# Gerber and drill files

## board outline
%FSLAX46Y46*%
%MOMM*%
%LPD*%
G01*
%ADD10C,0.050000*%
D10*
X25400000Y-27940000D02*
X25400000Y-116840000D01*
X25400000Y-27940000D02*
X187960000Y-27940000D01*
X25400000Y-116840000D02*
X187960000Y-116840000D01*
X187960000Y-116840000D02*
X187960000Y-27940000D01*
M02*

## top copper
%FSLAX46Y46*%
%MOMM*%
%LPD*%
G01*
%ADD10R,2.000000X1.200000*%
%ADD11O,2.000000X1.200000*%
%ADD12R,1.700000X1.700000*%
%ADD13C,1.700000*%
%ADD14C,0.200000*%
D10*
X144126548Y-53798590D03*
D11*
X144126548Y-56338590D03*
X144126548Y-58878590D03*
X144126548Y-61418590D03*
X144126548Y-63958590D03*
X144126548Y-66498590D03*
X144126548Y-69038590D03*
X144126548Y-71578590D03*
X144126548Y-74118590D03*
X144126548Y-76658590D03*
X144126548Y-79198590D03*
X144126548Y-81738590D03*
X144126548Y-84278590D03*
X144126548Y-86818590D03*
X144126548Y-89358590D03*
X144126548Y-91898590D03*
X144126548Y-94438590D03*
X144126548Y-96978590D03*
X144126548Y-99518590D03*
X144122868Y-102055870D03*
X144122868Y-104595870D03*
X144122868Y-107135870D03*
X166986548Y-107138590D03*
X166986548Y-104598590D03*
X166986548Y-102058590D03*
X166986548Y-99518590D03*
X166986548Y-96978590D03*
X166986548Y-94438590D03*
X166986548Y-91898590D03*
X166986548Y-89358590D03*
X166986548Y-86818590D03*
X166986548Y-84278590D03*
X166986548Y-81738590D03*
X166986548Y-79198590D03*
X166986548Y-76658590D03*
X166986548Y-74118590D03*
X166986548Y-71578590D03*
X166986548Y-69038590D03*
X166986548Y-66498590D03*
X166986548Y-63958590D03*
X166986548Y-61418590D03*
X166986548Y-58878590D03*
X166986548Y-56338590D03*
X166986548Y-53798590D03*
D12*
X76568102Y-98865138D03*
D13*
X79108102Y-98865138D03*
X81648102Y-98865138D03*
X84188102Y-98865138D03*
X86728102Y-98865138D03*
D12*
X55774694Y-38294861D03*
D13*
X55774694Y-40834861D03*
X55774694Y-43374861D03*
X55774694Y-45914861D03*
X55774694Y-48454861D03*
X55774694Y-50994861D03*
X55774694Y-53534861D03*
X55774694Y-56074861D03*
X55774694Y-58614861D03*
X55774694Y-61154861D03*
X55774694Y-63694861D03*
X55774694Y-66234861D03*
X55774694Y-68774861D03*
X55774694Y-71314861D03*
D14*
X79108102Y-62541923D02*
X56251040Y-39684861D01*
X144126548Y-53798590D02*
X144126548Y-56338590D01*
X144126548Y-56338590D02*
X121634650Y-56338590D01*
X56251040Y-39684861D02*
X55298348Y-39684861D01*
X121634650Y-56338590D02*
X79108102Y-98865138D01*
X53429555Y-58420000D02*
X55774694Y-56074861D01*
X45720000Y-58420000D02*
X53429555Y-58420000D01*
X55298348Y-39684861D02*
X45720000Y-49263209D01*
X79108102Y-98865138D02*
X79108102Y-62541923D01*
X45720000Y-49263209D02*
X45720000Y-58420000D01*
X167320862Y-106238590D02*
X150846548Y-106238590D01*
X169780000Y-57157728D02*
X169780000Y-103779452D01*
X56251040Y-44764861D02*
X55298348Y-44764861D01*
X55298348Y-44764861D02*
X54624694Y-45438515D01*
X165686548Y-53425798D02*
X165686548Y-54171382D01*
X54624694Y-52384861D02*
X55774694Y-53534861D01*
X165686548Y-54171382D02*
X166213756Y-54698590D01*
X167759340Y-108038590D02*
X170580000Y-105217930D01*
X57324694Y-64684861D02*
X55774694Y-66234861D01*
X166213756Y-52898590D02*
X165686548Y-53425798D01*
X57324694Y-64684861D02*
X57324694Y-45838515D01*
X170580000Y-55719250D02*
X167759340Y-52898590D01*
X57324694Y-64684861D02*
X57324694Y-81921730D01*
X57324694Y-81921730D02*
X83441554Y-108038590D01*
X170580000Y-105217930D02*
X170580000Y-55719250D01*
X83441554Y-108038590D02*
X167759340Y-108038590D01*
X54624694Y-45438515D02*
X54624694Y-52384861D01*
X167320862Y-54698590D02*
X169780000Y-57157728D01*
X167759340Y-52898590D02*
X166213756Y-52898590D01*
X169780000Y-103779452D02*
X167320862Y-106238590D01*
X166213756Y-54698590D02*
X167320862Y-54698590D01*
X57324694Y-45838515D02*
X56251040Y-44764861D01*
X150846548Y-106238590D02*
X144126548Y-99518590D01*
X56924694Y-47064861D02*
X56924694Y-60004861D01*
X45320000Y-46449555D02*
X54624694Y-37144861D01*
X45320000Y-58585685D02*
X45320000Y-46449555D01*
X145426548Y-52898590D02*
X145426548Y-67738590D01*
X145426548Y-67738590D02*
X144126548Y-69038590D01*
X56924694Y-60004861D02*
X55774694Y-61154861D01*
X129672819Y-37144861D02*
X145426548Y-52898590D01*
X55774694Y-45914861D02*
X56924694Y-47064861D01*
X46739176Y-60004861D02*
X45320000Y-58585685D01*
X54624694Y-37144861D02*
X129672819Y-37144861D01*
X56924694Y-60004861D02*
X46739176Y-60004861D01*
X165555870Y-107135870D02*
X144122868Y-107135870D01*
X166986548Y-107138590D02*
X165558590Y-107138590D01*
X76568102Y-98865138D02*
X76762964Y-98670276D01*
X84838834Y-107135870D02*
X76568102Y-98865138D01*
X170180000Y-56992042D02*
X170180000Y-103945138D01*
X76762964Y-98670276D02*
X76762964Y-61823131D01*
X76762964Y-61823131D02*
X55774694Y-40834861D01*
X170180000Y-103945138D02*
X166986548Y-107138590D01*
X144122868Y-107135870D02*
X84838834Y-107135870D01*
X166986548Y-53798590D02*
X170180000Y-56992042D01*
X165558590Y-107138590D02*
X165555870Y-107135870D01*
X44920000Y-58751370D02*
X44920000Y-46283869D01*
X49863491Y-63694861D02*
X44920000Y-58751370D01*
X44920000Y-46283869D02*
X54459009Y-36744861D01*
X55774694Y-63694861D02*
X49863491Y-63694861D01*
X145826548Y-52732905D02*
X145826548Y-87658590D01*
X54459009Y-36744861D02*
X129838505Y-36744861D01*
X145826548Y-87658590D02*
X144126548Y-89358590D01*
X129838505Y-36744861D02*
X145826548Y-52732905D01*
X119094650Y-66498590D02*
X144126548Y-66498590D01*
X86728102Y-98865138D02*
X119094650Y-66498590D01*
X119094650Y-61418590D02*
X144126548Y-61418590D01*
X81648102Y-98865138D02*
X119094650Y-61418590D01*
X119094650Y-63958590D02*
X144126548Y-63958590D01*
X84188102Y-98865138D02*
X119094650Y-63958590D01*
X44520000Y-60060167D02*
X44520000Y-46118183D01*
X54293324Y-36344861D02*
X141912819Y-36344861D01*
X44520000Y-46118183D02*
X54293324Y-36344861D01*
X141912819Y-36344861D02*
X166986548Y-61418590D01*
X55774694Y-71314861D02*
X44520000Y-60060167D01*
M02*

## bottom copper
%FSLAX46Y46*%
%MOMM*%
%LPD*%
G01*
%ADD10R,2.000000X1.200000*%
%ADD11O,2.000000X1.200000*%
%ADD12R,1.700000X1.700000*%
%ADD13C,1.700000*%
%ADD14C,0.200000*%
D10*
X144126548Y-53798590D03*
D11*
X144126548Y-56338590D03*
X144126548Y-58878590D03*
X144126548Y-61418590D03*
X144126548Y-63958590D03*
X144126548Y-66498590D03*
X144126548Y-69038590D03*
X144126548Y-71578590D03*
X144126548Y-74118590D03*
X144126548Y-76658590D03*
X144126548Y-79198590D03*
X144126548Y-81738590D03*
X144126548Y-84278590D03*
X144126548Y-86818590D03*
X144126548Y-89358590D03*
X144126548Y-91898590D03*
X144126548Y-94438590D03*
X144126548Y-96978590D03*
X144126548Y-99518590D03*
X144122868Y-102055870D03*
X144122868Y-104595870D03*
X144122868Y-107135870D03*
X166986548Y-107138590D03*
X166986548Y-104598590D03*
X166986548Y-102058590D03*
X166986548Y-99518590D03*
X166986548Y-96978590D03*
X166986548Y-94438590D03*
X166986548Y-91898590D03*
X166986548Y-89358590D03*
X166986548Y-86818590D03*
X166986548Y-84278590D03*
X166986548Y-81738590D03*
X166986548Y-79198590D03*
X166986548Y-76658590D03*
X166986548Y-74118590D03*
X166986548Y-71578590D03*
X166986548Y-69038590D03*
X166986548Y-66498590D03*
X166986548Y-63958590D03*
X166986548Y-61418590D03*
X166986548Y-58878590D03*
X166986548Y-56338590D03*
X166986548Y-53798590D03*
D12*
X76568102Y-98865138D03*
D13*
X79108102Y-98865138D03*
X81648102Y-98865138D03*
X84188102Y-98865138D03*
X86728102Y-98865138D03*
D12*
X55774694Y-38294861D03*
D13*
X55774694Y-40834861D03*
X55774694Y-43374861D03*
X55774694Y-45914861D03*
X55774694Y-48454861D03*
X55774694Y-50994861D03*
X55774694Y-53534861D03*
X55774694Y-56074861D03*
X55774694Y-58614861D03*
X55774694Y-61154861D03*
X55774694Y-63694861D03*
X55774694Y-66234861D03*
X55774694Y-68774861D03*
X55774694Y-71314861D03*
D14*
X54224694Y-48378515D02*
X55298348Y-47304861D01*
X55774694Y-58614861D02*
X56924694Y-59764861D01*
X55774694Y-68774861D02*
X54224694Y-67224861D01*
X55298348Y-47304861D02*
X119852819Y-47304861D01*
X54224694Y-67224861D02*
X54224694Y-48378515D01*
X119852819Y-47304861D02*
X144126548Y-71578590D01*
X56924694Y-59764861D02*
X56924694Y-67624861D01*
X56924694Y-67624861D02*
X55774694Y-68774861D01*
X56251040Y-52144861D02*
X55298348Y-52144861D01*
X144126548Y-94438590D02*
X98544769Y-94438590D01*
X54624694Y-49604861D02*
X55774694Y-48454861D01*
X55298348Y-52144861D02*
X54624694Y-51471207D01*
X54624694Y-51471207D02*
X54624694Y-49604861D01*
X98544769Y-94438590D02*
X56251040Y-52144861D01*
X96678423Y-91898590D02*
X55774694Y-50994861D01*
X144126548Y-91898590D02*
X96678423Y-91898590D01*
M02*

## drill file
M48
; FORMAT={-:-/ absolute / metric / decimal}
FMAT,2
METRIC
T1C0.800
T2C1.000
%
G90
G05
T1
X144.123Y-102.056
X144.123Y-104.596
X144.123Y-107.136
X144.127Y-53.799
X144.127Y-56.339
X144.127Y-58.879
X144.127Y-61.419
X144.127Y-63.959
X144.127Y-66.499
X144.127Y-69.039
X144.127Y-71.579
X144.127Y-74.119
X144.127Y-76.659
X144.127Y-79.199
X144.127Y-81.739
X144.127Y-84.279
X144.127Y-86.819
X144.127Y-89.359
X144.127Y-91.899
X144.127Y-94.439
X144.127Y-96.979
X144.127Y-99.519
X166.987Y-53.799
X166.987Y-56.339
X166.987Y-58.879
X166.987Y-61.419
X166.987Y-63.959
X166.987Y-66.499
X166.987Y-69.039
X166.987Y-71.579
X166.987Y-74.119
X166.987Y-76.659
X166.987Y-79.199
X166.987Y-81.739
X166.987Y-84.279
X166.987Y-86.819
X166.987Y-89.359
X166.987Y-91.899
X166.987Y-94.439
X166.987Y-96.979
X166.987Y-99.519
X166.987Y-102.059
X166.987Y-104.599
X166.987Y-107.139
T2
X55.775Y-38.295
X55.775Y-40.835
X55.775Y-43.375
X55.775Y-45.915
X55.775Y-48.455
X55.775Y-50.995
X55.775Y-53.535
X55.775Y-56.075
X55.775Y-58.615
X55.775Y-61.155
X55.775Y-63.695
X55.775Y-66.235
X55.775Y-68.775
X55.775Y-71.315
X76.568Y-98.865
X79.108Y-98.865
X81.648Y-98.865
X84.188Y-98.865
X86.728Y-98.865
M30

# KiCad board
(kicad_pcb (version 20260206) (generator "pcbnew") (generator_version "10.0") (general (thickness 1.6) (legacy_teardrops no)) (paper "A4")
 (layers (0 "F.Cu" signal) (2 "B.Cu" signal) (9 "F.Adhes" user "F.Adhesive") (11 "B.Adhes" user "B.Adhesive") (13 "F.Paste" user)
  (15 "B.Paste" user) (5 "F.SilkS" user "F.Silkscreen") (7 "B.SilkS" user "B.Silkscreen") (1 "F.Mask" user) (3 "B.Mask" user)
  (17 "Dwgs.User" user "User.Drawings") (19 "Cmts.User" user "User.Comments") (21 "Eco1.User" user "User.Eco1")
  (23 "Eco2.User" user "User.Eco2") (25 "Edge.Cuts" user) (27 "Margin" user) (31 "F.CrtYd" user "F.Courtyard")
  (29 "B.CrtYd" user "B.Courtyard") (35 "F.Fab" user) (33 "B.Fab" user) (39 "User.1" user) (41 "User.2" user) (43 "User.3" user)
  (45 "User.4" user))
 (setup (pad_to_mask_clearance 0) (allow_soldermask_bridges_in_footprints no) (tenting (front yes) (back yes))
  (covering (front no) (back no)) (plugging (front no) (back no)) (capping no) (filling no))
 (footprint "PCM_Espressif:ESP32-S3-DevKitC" (layer "F.Cu") (at 144.126548 53.79859)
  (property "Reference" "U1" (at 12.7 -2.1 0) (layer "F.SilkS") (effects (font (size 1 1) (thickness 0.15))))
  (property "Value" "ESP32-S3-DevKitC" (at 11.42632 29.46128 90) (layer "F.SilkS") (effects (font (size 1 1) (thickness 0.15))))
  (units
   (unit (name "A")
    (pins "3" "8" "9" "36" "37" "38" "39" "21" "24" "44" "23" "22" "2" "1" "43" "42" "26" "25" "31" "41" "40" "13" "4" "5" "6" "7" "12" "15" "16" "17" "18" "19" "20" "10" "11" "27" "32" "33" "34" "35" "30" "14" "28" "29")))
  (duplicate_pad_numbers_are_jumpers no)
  (pad "1" thru_hole rect (at 0 0 270) (size 1.2 2) (drill 0.8) (layers "*.Cu" "*.Mask") (remove_unused_layers no) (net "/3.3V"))
  (pad "2" thru_hole oval (at 0 2.54 270) (size 1.2 2) (drill 0.8) (layers "*.Cu" "*.Mask") (remove_unused_layers no) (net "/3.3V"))
  (pad "3" thru_hole oval (at 0 5.08 270) (size 1.2 2) (drill 0.8) (layers "*.Cu" "*.Mask") (remove_unused_layers no)
   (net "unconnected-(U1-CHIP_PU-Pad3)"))
  (pad "4" thru_hole oval (at 0 7.62 270) (size 1.2 2) (drill 0.8) (layers "*.Cu" "*.Mask") (remove_unused_layers no) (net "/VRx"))
  (pad "5" thru_hole oval (at 0 10.16 270) (size 1.2 2) (drill 0.8) (layers "*.Cu" "*.Mask") (remove_unused_layers no) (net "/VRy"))
  (pad "6" thru_hole oval (at 0 12.7 270) (size 1.2 2) (drill 0.8) (layers "*.Cu" "*.Mask") (remove_unused_layers no) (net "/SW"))
  (pad "7" thru_hole oval (at 0 15.24 270) (size 1.2 2) (drill 0.8) (layers "*.Cu" "*.Mask") (remove_unused_layers no) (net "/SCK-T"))
  (pad "8" thru_hole oval (at 0 17.78 270) (size 1.2 2) (drill 0.8) (layers "*.Cu" "*.Mask") (remove_unused_layers no) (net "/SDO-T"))
  (pad "9" thru_hole oval (at 0 20.32 270) (size 1.2 2) (drill 0.8) (layers "*.Cu" "*.Mask") (remove_unused_layers no)
   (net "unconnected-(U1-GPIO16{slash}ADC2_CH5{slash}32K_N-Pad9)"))
  (pad "10" thru_hole oval (at 0 22.86 270) (size 1.2 2) (drill 0.8) (layers "*.Cu" "*.Mask") (remove_unused_layers no)
   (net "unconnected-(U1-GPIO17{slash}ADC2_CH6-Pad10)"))
  (pad "11" thru_hole oval (at 0 25.4 270) (size 1.2 2) (drill 0.8) (layers "*.Cu" "*.Mask") (remove_unused_layers no)
   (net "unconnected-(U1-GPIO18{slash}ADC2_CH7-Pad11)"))
  (pad "12" thru_hole oval (at 0 27.94 270) (size 1.2 2) (drill 0.8) (layers "*.Cu" "*.Mask") (remove_unused_layers no)
   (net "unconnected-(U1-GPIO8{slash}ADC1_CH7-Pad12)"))
  (pad "13" thru_hole oval (at 0 30.48 270) (size 1.2 2) (drill 0.8) (layers "*.Cu" "*.Mask") (remove_unused_layers no)
   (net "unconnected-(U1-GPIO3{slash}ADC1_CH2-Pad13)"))
  (pad "14" thru_hole oval (at 0 33.02 270) (size 1.2 2) (drill 0.8) (layers "*.Cu" "*.Mask") (remove_unused_layers no)
   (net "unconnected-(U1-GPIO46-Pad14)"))
  (pad "15" thru_hole oval (at 0 35.56 270) (size 1.2 2) (drill 0.8) (layers "*.Cu" "*.Mask") (remove_unused_layers no) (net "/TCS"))
  (pad "16" thru_hole oval (at 0 38.1 270) (size 1.2 2) (drill 0.8) (layers "*.Cu" "*.Mask") (remove_unused_layers no) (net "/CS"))
  (pad "17" thru_hole oval (at 0 40.64 270) (size 1.2 2) (drill 0.8) (layers "*.Cu" "*.Mask") (remove_unused_layers no) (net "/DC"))
  (pad "18" thru_hole oval (at 0 43.18 270) (size 1.2 2) (drill 0.8) (layers "*.Cu" "*.Mask") (remove_unused_layers no)
   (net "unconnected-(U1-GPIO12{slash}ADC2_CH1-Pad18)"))
  (pad "19" thru_hole oval (at 0 45.72 270) (size 1.2 2) (drill 0.8) (layers "*.Cu" "*.Mask") (remove_unused_layers no) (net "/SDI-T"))
  (pad "20" thru_hole oval (at -0.00368 48.25728 270) (size 1.2 2) (drill 0.8) (layers "*.Cu" "*.Mask") (remove_unused_layers no)
   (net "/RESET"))
  (pad "21" thru_hole oval (at -0.00368 50.79728 270) (size 1.2 2) (drill 0.8) (layers "*.Cu" "*.Mask") (remove_unused_layers no)
   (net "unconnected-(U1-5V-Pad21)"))
  (pad "22" thru_hole oval (at -0.00368 53.33728 270) (size 1.2 2) (drill 0.8) (layers "*.Cu" "*.Mask") (remove_unused_layers no)
   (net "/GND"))
  (pad "23" thru_hole oval (at 22.86 53.34 270) (size 1.2 2) (drill 0.8) (layers "*.Cu" "*.Mask") (remove_unused_layers no) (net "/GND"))
  (pad "24" thru_hole oval (at 22.86 50.8 270) (size 1.2 2) (drill 0.8) (layers "*.Cu" "*.Mask") (remove_unused_layers no) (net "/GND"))
  (pad "25" thru_hole oval (at 22.86 48.26 270) (size 1.2 2) (drill 0.8) (layers "*.Cu" "*.Mask") (remove_unused_layers no)
   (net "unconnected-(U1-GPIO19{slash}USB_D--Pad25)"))
  (pad "26" thru_hole oval (at 22.86 45.72 270) (size 1.2 2) (drill 0.8) (layers "*.Cu" "*.Mask") (remove_unused_layers no)
   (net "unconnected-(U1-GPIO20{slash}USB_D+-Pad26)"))
  (pad "27" thru_hole oval (at 22.86 43.18 270) (size 1.2 2) (drill 0.8) (layers "*.Cu" "*.Mask") (remove_unused_layers no)
   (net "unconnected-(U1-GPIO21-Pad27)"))
  (pad "28" thru_hole oval (at 22.86 40.64 270) (size 1.2 2) (drill 0.8) (layers "*.Cu" "*.Mask") (remove_unused_layers no)
   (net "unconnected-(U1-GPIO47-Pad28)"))
  (pad "29" thru_hole oval (at 22.86 38.1 270) (size 1.2 2) (drill 0.8) (layers "*.Cu" "*.Mask") (remove_unused_layers no)
   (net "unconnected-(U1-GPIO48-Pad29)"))
  (pad "30" thru_hole oval (at 22.86 35.56 270) (size 1.2 2) (drill 0.8) (layers "*.Cu" "*.Mask") (remove_unused_layers no)
   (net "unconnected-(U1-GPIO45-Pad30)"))
  (pad "31" thru_hole oval (at 22.86 33.02 270) (size 1.2 2) (drill 0.8) (layers "*.Cu" "*.Mask") (remove_unused_layers no)
   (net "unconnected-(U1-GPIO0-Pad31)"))
  (pad "32" thru_hole oval (at 22.86 30.48 270) (size 1.2 2) (drill 0.8) (layers "*.Cu" "*.Mask") (remove_unused_layers no)
   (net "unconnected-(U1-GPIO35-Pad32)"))
  (pad "33" thru_hole oval (at 22.86 27.94 270) (size 1.2 2) (drill 0.8) (layers "*.Cu" "*.Mask") (remove_unused_layers no)
   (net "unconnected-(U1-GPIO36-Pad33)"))
  (pad "34" thru_hole oval (at 22.86 25.4 270) (size 1.2 2) (drill 0.8) (layers "*.Cu" "*.Mask") (remove_unused_layers no)
   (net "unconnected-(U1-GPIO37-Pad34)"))
  (pad "35" thru_hole oval (at 22.86 22.86 270) (size 1.2 2) (drill 0.8) (layers "*.Cu" "*.Mask") (remove_unused_layers no)
   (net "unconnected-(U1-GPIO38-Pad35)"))
  (pad "36" thru_hole oval (at 22.86 20.32 270) (size 1.2 2) (drill 0.8) (layers "*.Cu" "*.Mask") (remove_unused_layers no)
   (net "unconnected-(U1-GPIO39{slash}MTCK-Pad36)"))
  (pad "37" thru_hole oval (at 22.86 17.78 270) (size 1.2 2) (drill 0.8) (layers "*.Cu" "*.Mask") (remove_unused_layers no)
   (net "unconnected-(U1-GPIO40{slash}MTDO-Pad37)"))
  (pad "38" thru_hole oval (at 22.86 15.24 270) (size 1.2 2) (drill 0.8) (layers "*.Cu" "*.Mask") (remove_unused_layers no)
   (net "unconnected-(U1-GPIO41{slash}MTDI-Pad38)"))
  (pad "39" thru_hole oval (at 22.86 12.7 270) (size 1.2 2) (drill 0.8) (layers "*.Cu" "*.Mask") (remove_unused_layers no)
   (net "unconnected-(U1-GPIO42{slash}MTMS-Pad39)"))
  (pad "40" thru_hole oval (at 22.86 10.16 270) (size 1.2 2) (drill 0.8) (layers "*.Cu" "*.Mask") (remove_unused_layers no)
   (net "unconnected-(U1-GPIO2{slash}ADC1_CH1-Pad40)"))
  (pad "41" thru_hole oval (at 22.86 7.62 270) (size 1.2 2) (drill 0.8) (layers "*.Cu" "*.Mask") (remove_unused_layers no) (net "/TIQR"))
  (pad "42" thru_hole oval (at 22.86 5.08 270) (size 1.2 2) (drill 0.8) (layers "*.Cu" "*.Mask") (remove_unused_layers no)
   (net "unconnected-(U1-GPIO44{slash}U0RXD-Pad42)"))
  (pad "43" thru_hole oval (at 22.86 2.54 270) (size 1.2 2) (drill 0.8) (layers "*.Cu" "*.Mask") (remove_unused_layers no)
   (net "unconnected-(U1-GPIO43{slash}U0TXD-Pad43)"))
  (pad "44" thru_hole oval (at 22.86 0 270) (size 1.2 2) (drill 0.8) (layers "*.Cu" "*.Mask") (remove_unused_layers no) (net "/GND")))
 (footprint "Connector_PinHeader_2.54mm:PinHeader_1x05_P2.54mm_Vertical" (layer "F.Cu") (at 76.568102 98.865138 90)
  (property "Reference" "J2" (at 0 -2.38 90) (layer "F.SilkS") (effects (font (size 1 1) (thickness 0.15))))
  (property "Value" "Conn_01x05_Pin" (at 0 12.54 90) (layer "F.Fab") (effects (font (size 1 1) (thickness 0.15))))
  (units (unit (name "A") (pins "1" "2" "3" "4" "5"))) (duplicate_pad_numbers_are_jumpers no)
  (pad "1" thru_hole rect (at 0 0 90) (size 1.7 1.7) (drill 1) (layers "*.Cu" "*.Mask") (remove_unused_layers no) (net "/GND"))
  (pad "2" thru_hole circle (at 0 2.54 90) (size 1.7 1.7) (drill 1) (layers "*.Cu" "*.Mask") (remove_unused_layers no) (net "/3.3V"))
  (pad "3" thru_hole circle (at 0 5.08 90) (size 1.7 1.7) (drill 1) (layers "*.Cu" "*.Mask") (remove_unused_layers no) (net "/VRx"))
  (pad "4" thru_hole circle (at 0 7.62 90) (size 1.7 1.7) (drill 1) (layers "*.Cu" "*.Mask") (remove_unused_layers no) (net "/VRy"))
  (pad "5" thru_hole circle (at 0 10.16 90) (size 1.7 1.7) (drill 1) (layers "*.Cu" "*.Mask") (remove_unused_layers no) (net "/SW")))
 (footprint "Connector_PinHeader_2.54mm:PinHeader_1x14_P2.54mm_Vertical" (layer "F.Cu") (at 55.774694 38.294861)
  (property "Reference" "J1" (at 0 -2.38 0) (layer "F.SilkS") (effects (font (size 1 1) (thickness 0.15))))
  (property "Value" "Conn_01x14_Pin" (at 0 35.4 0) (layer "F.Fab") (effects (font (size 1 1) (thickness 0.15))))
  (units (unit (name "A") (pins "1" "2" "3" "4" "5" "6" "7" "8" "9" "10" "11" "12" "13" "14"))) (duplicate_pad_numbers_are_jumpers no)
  (pad "1" thru_hole rect (at 0 0) (size 1.7 1.7) (drill 1) (layers "*.Cu" "*.Mask") (remove_unused_layers no) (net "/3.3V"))
  (pad "2" thru_hole circle (at 0 2.54) (size 1.7 1.7) (drill 1) (layers "*.Cu" "*.Mask") (remove_unused_layers no) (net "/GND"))
  (pad "3" thru_hole circle (at 0 5.08) (size 1.7 1.7) (drill 1) (layers "*.Cu" "*.Mask") (remove_unused_layers no) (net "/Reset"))
  (pad "4" thru_hole circle (at 0 7.62) (size 1.7 1.7) (drill 1) (layers "*.Cu" "*.Mask") (remove_unused_layers no) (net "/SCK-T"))
  (pad "5" thru_hole circle (at 0 10.16) (size 1.7 1.7) (drill 1) (layers "*.Cu" "*.Mask") (remove_unused_layers no) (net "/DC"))
  (pad "6" thru_hole circle (at 0 12.7) (size 1.7 1.7) (drill 1) (layers "*.Cu" "*.Mask") (remove_unused_layers no) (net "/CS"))
  (pad "7" thru_hole circle (at 0 15.24) (size 1.7 1.7) (drill 1) (layers "*.Cu" "*.Mask") (remove_unused_layers no) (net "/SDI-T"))
  (pad "8" thru_hole circle (at 0 17.78) (size 1.7 1.7) (drill 1) (layers "*.Cu" "*.Mask") (remove_unused_layers no) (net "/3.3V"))
  (pad "9" thru_hole circle (at 0 20.32) (size 1.7 1.7) (drill 1) (layers "*.Cu" "*.Mask") (remove_unused_layers no) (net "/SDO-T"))
  (pad "10" thru_hole circle (at 0 22.86) (size 1.7 1.7) (drill 1) (layers "*.Cu" "*.Mask") (remove_unused_layers no) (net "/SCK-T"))
  (pad "11" thru_hole circle (at 0 25.4) (size 1.7 1.7) (drill 1) (layers "*.Cu" "*.Mask") (remove_unused_layers no) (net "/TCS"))
  (pad "12" thru_hole circle (at 0 27.94) (size 1.7 1.7) (drill 1) (layers "*.Cu" "*.Mask") (remove_unused_layers no) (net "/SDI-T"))
  (pad "13" thru_hole circle (at 0 30.48) (size 1.7 1.7) (drill 1) (layers "*.Cu" "*.Mask") (remove_unused_layers no) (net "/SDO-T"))
  (pad "14" thru_hole circle (at 0 33.02) (size 1.7 1.7) (drill 1) (layers "*.Cu" "*.Mask") (remove_unused_layers no) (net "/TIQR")))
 (gr_line (start 25.4 27.94) (end 25.4 116.84) (stroke (width 0.05) (type default)) (layer "Edge.Cuts"))
 (gr_line (start 25.4 27.94) (end 187.96 27.94) (stroke (width 0.05) (type default)) (layer "Edge.Cuts"))
 (gr_line (start 25.4 116.84) (end 187.96 116.84) (stroke (width 0.05) (type default)) (layer "Edge.Cuts"))
 (gr_line (start 187.96 116.84) (end 187.96 27.94) (stroke (width 0.05) (type default)) (layer "Edge.Cuts"))
 (segment (start 54.224694 48.378515) (end 55.298348 47.304861) (width 0.2) (layer "B.Cu") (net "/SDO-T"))
 (segment (start 55.774694 58.614861) (end 56.924694 59.764861) (width 0.2) (layer "B.Cu") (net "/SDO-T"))
 (segment (start 55.774694 68.774861) (end 54.224694 67.224861) (width 0.2) (layer "B.Cu") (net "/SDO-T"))
 (segment (start 55.298348 47.304861) (end 119.852819 47.304861) (width 0.2) (layer "B.Cu") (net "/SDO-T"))
 (segment (start 54.224694 67.224861) (end 54.224694 48.378515) (width 0.2) (layer "B.Cu") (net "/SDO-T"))
 (segment (start 119.852819 47.304861) (end 144.126548 71.57859) (width 0.2) (layer "B.Cu") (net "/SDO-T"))
 (segment (start 56.924694 59.764861) (end 56.924694 67.624861) (width 0.2) (layer "B.Cu") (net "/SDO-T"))
 (segment (start 56.924694 67.624861) (end 55.774694 68.774861) (width 0.2) (layer "B.Cu") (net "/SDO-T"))
 (segment (start 79.108102 62.541923) (end 56.25104 39.684861) (width 0.2) (layer "F.Cu") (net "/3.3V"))
 (segment (start 144.126548 53.79859) (end 144.126548 56.33859) (width 0.2) (layer "F.Cu") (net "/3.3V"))
 (segment (start 144.126548 56.33859) (end 121.63465 56.33859) (width 0.2) (layer "F.Cu") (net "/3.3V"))
 (segment (start 56.25104 39.684861) (end 55.298348 39.684861) (width 0.2) (layer "F.Cu") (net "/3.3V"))
 (segment (start 121.63465 56.33859) (end 79.108102 98.865138) (width 0.2) (layer "F.Cu") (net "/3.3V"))
 (segment (start 53.429555 58.42) (end 55.774694 56.074861) (width 0.2) (layer "F.Cu") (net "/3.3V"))
 (segment (start 45.72 58.42) (end 53.429555 58.42) (width 0.2) (layer "F.Cu") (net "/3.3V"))
 (segment (start 55.298348 39.684861) (end 45.72 49.263209) (width 0.2) (layer "F.Cu") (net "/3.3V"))
 (segment (start 79.108102 98.865138) (end 79.108102 62.541923) (width 0.2) (layer "F.Cu") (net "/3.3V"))
 (segment (start 45.72 49.263209) (end 45.72 58.42) (width 0.2) (layer "F.Cu") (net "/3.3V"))
 (segment (start 167.320862 106.23859) (end 150.846548 106.23859) (width 0.2) (layer "F.Cu") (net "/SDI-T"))
 (segment (start 169.78 57.157728) (end 169.78 103.779452) (width 0.2) (layer "F.Cu") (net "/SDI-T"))
 (segment (start 56.25104 44.764861) (end 55.298348 44.764861) (width 0.2) (layer "F.Cu") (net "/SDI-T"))
 (segment (start 55.298348 44.764861) (end 54.624694 45.438515) (width 0.2) (layer "F.Cu") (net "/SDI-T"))
 (segment (start 165.686548 53.425798) (end 165.686548 54.171382) (width 0.2) (layer "F.Cu") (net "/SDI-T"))
 (segment (start 54.624694 52.384861) (end 55.774694 53.534861) (width 0.2) (layer "F.Cu") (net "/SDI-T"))
 (segment (start 165.686548 54.171382) (end 166.213756 54.69859) (width 0.2) (layer "F.Cu") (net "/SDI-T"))
 (segment (start 167.75934 108.03859) (end 170.58 105.21793) (width 0.2) (layer "F.Cu") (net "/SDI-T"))
 (segment (start 57.324694 64.684861) (end 55.774694 66.234861) (width 0.2) (layer "F.Cu") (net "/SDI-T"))
 (segment (start 166.213756 52.89859) (end 165.686548 53.425798) (width 0.2) (layer "F.Cu") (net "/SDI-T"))
 (segment (start 57.324694 64.684861) (end 57.324694 45.838515) (width 0.2) (layer "F.Cu") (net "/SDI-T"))
 (segment (start 170.58 55.71925) (end 167.75934 52.89859) (width 0.2) (layer "F.Cu") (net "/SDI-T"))
 (segment (start 57.324694 64.684861) (end 57.324694 81.92173) (width 0.2) (layer "F.Cu") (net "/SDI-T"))
 (segment (start 57.324694 81.92173) (end 83.441554 108.03859) (width 0.2) (layer "F.Cu") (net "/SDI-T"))
 (segment (start 170.58 105.21793) (end 170.58 55.71925) (width 0.2) (layer "F.Cu") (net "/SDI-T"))
 (segment (start 83.441554 108.03859) (end 167.75934 108.03859) (width 0.2) (layer "F.Cu") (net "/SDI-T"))
 (segment (start 54.624694 45.438515) (end 54.624694 52.384861) (width 0.2) (layer "F.Cu") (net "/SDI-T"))
 (segment (start 167.320862 54.69859) (end 169.78 57.157728) (width 0.2) (layer "F.Cu") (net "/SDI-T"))
 (segment (start 167.75934 52.89859) (end 166.213756 52.89859) (width 0.2) (layer "F.Cu") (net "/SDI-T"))
 (segment (start 169.78 103.779452) (end 167.320862 106.23859) (width 0.2) (layer "F.Cu") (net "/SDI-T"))
 (segment (start 166.213756 54.69859) (end 167.320862 54.69859) (width 0.2) (layer "F.Cu") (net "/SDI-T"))
 (segment (start 57.324694 45.838515) (end 56.25104 44.764861) (width 0.2) (layer "F.Cu") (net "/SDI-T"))
 (segment (start 150.846548 106.23859) (end 144.126548 99.51859) (width 0.2) (layer "F.Cu") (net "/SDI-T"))
 (segment (start 56.924694 47.064861) (end 56.924694 60.004861) (width 0.2) (layer "F.Cu") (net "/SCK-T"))
 (segment (start 45.32 46.449555) (end 54.624694 37.144861) (width 0.2) (layer "F.Cu") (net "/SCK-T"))
 (segment (start 45.32 58.585685) (end 45.32 46.449555) (width 0.2) (layer "F.Cu") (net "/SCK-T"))
 (segment (start 145.426548 52.89859) (end 145.426548 67.73859) (width 0.2) (layer "F.Cu") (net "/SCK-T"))
 (segment (start 145.426548 67.73859) (end 144.126548 69.03859) (width 0.2) (layer "F.Cu") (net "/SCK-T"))
 (segment (start 56.924694 60.004861) (end 55.774694 61.154861) (width 0.2) (layer "F.Cu") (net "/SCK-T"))
 (segment (start 129.672819 37.144861) (end 145.426548 52.89859) (width 0.2) (layer "F.Cu") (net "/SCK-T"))
 (segment (start 55.774694 45.914861) (end 56.924694 47.064861) (width 0.2) (layer "F.Cu") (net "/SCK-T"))
 (segment (start 46.739176 60.004861) (end 45.32 58.585685) (width 0.2) (layer "F.Cu") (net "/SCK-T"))
 (segment (start 54.624694 37.144861) (end 129.672819 37.144861) (width 0.2) (layer "F.Cu") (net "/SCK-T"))
 (segment (start 56.924694 60.004861) (end 46.739176 60.004861) (width 0.2) (layer "F.Cu") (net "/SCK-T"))
 (segment (start 56.25104 52.144861) (end 55.298348 52.144861) (width 0.2) (layer "B.Cu") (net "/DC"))
 (segment (start 144.126548 94.43859) (end 98.544769 94.43859) (width 0.2) (layer "B.Cu") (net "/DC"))
 (segment (start 54.624694 49.604861) (end 55.774694 48.454861) (width 0.2) (layer "B.Cu") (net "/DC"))
 (segment (start 55.298348 52.144861) (end 54.624694 51.471207) (width 0.2) (layer "B.Cu") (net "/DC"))
 (segment (start 54.624694 51.471207) (end 54.624694 49.604861) (width 0.2) (layer "B.Cu") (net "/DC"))
 (segment (start 98.544769 94.43859) (end 56.25104 52.144861) (width 0.2) (layer "B.Cu") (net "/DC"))
 (segment (start 96.678423 91.89859) (end 55.774694 50.994861) (width 0.2) (layer "B.Cu") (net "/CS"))
 (segment (start 144.126548 91.89859) (end 96.678423 91.89859) (width 0.2) (layer "B.Cu") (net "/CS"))
 (segment (start 165.55587 107.13587) (end 144.122868 107.13587) (width 0.2) (layer "F.Cu") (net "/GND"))
 (segment (start 166.986548 107.13859) (end 165.55859 107.13859) (width 0.2) (layer "F.Cu") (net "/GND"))
 (segment (start 76.568102 98.865138) (end 76.762964 98.670276) (width 0.2) (layer "F.Cu") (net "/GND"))
 (segment (start 84.838834 107.13587) (end 76.568102 98.865138) (width 0.2) (layer "F.Cu") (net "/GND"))
 (segment (start 170.18 56.992042) (end 170.18 103.945138) (width 0.2) (layer "F.Cu") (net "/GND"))
 (segment (start 76.762964 98.670276) (end 76.762964 61.823131) (width 0.2) (layer "F.Cu") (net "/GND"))
 (segment (start 76.762964 61.823131) (end 55.774694 40.834861) (width 0.2) (layer "F.Cu") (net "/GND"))
 (segment (start 170.18 103.945138) (end 166.986548 107.13859) (width 0.2) (layer "F.Cu") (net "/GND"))
 (segment (start 144.122868 107.13587) (end 84.838834 107.13587) (width 0.2) (layer "F.Cu") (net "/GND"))
 (segment (start 166.986548 53.79859) (end 170.18 56.992042) (width 0.2) (layer "F.Cu") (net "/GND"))
 (segment (start 165.55859 107.13859) (end 165.55587 107.13587) (width 0.2) (layer "F.Cu") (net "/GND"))
 (segment (start 44.92 58.75137) (end 44.92 46.283869) (width 0.2) (layer "F.Cu") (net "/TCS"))
 (segment (start 49.863491 63.694861) (end 44.92 58.75137) (width 0.2) (layer "F.Cu") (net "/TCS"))
 (segment (start 44.92 46.283869) (end 54.459009 36.744861) (width 0.2) (layer "F.Cu") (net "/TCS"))
 (segment (start 55.774694 63.694861) (end 49.863491 63.694861) (width 0.2) (layer "F.Cu") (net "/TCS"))
 (segment (start 145.826548 52.732905) (end 145.826548 87.65859) (width 0.2) (layer "F.Cu") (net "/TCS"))
 (segment (start 54.459009 36.744861) (end 129.838505 36.744861) (width 0.2) (layer "F.Cu") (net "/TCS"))
 (segment (start 145.826548 87.65859) (end 144.126548 89.35859) (width 0.2) (layer "F.Cu") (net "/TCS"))
 (segment (start 129.838505 36.744861) (end 145.826548 52.732905) (width 0.2) (layer "F.Cu") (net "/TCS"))
 (segment (start 119.09465 66.49859) (end 144.126548 66.49859) (width 0.2) (layer "F.Cu") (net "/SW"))
 (segment (start 86.728102 98.865138) (end 119.09465 66.49859) (width 0.2) (layer "F.Cu") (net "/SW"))
 (segment (start 119.09465 61.41859) (end 144.126548 61.41859) (width 0.2) (layer "F.Cu") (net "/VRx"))
 (segment (start 81.648102 98.865138) (end 119.09465 61.41859) (width 0.2) (layer "F.Cu") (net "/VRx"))
 (segment (start 119.09465 63.95859) (end 144.126548 63.95859) (width 0.2) (layer "F.Cu") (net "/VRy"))
 (segment (start 84.188102 98.865138) (end 119.09465 63.95859) (width 0.2) (layer "F.Cu") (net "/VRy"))
 (segment (start 44.52 60.060167) (end 44.52 46.118183) (width 0.2) (layer "F.Cu") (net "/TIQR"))
 (segment (start 54.293324 36.344861) (end 141.912819 36.344861) (width 0.2) (layer "F.Cu") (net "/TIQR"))
 (segment (start 44.52 46.118183) (end 54.293324 36.344861) (width 0.2) (layer "F.Cu") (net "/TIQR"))
 (segment (start 141.912819 36.344861) (end 166.986548 61.41859) (width 0.2) (layer "F.Cu") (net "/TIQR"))
 (segment (start 55.774694 71.314861) (end 44.52 60.060167) (width 0.2) (layer "F.Cu") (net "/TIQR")))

